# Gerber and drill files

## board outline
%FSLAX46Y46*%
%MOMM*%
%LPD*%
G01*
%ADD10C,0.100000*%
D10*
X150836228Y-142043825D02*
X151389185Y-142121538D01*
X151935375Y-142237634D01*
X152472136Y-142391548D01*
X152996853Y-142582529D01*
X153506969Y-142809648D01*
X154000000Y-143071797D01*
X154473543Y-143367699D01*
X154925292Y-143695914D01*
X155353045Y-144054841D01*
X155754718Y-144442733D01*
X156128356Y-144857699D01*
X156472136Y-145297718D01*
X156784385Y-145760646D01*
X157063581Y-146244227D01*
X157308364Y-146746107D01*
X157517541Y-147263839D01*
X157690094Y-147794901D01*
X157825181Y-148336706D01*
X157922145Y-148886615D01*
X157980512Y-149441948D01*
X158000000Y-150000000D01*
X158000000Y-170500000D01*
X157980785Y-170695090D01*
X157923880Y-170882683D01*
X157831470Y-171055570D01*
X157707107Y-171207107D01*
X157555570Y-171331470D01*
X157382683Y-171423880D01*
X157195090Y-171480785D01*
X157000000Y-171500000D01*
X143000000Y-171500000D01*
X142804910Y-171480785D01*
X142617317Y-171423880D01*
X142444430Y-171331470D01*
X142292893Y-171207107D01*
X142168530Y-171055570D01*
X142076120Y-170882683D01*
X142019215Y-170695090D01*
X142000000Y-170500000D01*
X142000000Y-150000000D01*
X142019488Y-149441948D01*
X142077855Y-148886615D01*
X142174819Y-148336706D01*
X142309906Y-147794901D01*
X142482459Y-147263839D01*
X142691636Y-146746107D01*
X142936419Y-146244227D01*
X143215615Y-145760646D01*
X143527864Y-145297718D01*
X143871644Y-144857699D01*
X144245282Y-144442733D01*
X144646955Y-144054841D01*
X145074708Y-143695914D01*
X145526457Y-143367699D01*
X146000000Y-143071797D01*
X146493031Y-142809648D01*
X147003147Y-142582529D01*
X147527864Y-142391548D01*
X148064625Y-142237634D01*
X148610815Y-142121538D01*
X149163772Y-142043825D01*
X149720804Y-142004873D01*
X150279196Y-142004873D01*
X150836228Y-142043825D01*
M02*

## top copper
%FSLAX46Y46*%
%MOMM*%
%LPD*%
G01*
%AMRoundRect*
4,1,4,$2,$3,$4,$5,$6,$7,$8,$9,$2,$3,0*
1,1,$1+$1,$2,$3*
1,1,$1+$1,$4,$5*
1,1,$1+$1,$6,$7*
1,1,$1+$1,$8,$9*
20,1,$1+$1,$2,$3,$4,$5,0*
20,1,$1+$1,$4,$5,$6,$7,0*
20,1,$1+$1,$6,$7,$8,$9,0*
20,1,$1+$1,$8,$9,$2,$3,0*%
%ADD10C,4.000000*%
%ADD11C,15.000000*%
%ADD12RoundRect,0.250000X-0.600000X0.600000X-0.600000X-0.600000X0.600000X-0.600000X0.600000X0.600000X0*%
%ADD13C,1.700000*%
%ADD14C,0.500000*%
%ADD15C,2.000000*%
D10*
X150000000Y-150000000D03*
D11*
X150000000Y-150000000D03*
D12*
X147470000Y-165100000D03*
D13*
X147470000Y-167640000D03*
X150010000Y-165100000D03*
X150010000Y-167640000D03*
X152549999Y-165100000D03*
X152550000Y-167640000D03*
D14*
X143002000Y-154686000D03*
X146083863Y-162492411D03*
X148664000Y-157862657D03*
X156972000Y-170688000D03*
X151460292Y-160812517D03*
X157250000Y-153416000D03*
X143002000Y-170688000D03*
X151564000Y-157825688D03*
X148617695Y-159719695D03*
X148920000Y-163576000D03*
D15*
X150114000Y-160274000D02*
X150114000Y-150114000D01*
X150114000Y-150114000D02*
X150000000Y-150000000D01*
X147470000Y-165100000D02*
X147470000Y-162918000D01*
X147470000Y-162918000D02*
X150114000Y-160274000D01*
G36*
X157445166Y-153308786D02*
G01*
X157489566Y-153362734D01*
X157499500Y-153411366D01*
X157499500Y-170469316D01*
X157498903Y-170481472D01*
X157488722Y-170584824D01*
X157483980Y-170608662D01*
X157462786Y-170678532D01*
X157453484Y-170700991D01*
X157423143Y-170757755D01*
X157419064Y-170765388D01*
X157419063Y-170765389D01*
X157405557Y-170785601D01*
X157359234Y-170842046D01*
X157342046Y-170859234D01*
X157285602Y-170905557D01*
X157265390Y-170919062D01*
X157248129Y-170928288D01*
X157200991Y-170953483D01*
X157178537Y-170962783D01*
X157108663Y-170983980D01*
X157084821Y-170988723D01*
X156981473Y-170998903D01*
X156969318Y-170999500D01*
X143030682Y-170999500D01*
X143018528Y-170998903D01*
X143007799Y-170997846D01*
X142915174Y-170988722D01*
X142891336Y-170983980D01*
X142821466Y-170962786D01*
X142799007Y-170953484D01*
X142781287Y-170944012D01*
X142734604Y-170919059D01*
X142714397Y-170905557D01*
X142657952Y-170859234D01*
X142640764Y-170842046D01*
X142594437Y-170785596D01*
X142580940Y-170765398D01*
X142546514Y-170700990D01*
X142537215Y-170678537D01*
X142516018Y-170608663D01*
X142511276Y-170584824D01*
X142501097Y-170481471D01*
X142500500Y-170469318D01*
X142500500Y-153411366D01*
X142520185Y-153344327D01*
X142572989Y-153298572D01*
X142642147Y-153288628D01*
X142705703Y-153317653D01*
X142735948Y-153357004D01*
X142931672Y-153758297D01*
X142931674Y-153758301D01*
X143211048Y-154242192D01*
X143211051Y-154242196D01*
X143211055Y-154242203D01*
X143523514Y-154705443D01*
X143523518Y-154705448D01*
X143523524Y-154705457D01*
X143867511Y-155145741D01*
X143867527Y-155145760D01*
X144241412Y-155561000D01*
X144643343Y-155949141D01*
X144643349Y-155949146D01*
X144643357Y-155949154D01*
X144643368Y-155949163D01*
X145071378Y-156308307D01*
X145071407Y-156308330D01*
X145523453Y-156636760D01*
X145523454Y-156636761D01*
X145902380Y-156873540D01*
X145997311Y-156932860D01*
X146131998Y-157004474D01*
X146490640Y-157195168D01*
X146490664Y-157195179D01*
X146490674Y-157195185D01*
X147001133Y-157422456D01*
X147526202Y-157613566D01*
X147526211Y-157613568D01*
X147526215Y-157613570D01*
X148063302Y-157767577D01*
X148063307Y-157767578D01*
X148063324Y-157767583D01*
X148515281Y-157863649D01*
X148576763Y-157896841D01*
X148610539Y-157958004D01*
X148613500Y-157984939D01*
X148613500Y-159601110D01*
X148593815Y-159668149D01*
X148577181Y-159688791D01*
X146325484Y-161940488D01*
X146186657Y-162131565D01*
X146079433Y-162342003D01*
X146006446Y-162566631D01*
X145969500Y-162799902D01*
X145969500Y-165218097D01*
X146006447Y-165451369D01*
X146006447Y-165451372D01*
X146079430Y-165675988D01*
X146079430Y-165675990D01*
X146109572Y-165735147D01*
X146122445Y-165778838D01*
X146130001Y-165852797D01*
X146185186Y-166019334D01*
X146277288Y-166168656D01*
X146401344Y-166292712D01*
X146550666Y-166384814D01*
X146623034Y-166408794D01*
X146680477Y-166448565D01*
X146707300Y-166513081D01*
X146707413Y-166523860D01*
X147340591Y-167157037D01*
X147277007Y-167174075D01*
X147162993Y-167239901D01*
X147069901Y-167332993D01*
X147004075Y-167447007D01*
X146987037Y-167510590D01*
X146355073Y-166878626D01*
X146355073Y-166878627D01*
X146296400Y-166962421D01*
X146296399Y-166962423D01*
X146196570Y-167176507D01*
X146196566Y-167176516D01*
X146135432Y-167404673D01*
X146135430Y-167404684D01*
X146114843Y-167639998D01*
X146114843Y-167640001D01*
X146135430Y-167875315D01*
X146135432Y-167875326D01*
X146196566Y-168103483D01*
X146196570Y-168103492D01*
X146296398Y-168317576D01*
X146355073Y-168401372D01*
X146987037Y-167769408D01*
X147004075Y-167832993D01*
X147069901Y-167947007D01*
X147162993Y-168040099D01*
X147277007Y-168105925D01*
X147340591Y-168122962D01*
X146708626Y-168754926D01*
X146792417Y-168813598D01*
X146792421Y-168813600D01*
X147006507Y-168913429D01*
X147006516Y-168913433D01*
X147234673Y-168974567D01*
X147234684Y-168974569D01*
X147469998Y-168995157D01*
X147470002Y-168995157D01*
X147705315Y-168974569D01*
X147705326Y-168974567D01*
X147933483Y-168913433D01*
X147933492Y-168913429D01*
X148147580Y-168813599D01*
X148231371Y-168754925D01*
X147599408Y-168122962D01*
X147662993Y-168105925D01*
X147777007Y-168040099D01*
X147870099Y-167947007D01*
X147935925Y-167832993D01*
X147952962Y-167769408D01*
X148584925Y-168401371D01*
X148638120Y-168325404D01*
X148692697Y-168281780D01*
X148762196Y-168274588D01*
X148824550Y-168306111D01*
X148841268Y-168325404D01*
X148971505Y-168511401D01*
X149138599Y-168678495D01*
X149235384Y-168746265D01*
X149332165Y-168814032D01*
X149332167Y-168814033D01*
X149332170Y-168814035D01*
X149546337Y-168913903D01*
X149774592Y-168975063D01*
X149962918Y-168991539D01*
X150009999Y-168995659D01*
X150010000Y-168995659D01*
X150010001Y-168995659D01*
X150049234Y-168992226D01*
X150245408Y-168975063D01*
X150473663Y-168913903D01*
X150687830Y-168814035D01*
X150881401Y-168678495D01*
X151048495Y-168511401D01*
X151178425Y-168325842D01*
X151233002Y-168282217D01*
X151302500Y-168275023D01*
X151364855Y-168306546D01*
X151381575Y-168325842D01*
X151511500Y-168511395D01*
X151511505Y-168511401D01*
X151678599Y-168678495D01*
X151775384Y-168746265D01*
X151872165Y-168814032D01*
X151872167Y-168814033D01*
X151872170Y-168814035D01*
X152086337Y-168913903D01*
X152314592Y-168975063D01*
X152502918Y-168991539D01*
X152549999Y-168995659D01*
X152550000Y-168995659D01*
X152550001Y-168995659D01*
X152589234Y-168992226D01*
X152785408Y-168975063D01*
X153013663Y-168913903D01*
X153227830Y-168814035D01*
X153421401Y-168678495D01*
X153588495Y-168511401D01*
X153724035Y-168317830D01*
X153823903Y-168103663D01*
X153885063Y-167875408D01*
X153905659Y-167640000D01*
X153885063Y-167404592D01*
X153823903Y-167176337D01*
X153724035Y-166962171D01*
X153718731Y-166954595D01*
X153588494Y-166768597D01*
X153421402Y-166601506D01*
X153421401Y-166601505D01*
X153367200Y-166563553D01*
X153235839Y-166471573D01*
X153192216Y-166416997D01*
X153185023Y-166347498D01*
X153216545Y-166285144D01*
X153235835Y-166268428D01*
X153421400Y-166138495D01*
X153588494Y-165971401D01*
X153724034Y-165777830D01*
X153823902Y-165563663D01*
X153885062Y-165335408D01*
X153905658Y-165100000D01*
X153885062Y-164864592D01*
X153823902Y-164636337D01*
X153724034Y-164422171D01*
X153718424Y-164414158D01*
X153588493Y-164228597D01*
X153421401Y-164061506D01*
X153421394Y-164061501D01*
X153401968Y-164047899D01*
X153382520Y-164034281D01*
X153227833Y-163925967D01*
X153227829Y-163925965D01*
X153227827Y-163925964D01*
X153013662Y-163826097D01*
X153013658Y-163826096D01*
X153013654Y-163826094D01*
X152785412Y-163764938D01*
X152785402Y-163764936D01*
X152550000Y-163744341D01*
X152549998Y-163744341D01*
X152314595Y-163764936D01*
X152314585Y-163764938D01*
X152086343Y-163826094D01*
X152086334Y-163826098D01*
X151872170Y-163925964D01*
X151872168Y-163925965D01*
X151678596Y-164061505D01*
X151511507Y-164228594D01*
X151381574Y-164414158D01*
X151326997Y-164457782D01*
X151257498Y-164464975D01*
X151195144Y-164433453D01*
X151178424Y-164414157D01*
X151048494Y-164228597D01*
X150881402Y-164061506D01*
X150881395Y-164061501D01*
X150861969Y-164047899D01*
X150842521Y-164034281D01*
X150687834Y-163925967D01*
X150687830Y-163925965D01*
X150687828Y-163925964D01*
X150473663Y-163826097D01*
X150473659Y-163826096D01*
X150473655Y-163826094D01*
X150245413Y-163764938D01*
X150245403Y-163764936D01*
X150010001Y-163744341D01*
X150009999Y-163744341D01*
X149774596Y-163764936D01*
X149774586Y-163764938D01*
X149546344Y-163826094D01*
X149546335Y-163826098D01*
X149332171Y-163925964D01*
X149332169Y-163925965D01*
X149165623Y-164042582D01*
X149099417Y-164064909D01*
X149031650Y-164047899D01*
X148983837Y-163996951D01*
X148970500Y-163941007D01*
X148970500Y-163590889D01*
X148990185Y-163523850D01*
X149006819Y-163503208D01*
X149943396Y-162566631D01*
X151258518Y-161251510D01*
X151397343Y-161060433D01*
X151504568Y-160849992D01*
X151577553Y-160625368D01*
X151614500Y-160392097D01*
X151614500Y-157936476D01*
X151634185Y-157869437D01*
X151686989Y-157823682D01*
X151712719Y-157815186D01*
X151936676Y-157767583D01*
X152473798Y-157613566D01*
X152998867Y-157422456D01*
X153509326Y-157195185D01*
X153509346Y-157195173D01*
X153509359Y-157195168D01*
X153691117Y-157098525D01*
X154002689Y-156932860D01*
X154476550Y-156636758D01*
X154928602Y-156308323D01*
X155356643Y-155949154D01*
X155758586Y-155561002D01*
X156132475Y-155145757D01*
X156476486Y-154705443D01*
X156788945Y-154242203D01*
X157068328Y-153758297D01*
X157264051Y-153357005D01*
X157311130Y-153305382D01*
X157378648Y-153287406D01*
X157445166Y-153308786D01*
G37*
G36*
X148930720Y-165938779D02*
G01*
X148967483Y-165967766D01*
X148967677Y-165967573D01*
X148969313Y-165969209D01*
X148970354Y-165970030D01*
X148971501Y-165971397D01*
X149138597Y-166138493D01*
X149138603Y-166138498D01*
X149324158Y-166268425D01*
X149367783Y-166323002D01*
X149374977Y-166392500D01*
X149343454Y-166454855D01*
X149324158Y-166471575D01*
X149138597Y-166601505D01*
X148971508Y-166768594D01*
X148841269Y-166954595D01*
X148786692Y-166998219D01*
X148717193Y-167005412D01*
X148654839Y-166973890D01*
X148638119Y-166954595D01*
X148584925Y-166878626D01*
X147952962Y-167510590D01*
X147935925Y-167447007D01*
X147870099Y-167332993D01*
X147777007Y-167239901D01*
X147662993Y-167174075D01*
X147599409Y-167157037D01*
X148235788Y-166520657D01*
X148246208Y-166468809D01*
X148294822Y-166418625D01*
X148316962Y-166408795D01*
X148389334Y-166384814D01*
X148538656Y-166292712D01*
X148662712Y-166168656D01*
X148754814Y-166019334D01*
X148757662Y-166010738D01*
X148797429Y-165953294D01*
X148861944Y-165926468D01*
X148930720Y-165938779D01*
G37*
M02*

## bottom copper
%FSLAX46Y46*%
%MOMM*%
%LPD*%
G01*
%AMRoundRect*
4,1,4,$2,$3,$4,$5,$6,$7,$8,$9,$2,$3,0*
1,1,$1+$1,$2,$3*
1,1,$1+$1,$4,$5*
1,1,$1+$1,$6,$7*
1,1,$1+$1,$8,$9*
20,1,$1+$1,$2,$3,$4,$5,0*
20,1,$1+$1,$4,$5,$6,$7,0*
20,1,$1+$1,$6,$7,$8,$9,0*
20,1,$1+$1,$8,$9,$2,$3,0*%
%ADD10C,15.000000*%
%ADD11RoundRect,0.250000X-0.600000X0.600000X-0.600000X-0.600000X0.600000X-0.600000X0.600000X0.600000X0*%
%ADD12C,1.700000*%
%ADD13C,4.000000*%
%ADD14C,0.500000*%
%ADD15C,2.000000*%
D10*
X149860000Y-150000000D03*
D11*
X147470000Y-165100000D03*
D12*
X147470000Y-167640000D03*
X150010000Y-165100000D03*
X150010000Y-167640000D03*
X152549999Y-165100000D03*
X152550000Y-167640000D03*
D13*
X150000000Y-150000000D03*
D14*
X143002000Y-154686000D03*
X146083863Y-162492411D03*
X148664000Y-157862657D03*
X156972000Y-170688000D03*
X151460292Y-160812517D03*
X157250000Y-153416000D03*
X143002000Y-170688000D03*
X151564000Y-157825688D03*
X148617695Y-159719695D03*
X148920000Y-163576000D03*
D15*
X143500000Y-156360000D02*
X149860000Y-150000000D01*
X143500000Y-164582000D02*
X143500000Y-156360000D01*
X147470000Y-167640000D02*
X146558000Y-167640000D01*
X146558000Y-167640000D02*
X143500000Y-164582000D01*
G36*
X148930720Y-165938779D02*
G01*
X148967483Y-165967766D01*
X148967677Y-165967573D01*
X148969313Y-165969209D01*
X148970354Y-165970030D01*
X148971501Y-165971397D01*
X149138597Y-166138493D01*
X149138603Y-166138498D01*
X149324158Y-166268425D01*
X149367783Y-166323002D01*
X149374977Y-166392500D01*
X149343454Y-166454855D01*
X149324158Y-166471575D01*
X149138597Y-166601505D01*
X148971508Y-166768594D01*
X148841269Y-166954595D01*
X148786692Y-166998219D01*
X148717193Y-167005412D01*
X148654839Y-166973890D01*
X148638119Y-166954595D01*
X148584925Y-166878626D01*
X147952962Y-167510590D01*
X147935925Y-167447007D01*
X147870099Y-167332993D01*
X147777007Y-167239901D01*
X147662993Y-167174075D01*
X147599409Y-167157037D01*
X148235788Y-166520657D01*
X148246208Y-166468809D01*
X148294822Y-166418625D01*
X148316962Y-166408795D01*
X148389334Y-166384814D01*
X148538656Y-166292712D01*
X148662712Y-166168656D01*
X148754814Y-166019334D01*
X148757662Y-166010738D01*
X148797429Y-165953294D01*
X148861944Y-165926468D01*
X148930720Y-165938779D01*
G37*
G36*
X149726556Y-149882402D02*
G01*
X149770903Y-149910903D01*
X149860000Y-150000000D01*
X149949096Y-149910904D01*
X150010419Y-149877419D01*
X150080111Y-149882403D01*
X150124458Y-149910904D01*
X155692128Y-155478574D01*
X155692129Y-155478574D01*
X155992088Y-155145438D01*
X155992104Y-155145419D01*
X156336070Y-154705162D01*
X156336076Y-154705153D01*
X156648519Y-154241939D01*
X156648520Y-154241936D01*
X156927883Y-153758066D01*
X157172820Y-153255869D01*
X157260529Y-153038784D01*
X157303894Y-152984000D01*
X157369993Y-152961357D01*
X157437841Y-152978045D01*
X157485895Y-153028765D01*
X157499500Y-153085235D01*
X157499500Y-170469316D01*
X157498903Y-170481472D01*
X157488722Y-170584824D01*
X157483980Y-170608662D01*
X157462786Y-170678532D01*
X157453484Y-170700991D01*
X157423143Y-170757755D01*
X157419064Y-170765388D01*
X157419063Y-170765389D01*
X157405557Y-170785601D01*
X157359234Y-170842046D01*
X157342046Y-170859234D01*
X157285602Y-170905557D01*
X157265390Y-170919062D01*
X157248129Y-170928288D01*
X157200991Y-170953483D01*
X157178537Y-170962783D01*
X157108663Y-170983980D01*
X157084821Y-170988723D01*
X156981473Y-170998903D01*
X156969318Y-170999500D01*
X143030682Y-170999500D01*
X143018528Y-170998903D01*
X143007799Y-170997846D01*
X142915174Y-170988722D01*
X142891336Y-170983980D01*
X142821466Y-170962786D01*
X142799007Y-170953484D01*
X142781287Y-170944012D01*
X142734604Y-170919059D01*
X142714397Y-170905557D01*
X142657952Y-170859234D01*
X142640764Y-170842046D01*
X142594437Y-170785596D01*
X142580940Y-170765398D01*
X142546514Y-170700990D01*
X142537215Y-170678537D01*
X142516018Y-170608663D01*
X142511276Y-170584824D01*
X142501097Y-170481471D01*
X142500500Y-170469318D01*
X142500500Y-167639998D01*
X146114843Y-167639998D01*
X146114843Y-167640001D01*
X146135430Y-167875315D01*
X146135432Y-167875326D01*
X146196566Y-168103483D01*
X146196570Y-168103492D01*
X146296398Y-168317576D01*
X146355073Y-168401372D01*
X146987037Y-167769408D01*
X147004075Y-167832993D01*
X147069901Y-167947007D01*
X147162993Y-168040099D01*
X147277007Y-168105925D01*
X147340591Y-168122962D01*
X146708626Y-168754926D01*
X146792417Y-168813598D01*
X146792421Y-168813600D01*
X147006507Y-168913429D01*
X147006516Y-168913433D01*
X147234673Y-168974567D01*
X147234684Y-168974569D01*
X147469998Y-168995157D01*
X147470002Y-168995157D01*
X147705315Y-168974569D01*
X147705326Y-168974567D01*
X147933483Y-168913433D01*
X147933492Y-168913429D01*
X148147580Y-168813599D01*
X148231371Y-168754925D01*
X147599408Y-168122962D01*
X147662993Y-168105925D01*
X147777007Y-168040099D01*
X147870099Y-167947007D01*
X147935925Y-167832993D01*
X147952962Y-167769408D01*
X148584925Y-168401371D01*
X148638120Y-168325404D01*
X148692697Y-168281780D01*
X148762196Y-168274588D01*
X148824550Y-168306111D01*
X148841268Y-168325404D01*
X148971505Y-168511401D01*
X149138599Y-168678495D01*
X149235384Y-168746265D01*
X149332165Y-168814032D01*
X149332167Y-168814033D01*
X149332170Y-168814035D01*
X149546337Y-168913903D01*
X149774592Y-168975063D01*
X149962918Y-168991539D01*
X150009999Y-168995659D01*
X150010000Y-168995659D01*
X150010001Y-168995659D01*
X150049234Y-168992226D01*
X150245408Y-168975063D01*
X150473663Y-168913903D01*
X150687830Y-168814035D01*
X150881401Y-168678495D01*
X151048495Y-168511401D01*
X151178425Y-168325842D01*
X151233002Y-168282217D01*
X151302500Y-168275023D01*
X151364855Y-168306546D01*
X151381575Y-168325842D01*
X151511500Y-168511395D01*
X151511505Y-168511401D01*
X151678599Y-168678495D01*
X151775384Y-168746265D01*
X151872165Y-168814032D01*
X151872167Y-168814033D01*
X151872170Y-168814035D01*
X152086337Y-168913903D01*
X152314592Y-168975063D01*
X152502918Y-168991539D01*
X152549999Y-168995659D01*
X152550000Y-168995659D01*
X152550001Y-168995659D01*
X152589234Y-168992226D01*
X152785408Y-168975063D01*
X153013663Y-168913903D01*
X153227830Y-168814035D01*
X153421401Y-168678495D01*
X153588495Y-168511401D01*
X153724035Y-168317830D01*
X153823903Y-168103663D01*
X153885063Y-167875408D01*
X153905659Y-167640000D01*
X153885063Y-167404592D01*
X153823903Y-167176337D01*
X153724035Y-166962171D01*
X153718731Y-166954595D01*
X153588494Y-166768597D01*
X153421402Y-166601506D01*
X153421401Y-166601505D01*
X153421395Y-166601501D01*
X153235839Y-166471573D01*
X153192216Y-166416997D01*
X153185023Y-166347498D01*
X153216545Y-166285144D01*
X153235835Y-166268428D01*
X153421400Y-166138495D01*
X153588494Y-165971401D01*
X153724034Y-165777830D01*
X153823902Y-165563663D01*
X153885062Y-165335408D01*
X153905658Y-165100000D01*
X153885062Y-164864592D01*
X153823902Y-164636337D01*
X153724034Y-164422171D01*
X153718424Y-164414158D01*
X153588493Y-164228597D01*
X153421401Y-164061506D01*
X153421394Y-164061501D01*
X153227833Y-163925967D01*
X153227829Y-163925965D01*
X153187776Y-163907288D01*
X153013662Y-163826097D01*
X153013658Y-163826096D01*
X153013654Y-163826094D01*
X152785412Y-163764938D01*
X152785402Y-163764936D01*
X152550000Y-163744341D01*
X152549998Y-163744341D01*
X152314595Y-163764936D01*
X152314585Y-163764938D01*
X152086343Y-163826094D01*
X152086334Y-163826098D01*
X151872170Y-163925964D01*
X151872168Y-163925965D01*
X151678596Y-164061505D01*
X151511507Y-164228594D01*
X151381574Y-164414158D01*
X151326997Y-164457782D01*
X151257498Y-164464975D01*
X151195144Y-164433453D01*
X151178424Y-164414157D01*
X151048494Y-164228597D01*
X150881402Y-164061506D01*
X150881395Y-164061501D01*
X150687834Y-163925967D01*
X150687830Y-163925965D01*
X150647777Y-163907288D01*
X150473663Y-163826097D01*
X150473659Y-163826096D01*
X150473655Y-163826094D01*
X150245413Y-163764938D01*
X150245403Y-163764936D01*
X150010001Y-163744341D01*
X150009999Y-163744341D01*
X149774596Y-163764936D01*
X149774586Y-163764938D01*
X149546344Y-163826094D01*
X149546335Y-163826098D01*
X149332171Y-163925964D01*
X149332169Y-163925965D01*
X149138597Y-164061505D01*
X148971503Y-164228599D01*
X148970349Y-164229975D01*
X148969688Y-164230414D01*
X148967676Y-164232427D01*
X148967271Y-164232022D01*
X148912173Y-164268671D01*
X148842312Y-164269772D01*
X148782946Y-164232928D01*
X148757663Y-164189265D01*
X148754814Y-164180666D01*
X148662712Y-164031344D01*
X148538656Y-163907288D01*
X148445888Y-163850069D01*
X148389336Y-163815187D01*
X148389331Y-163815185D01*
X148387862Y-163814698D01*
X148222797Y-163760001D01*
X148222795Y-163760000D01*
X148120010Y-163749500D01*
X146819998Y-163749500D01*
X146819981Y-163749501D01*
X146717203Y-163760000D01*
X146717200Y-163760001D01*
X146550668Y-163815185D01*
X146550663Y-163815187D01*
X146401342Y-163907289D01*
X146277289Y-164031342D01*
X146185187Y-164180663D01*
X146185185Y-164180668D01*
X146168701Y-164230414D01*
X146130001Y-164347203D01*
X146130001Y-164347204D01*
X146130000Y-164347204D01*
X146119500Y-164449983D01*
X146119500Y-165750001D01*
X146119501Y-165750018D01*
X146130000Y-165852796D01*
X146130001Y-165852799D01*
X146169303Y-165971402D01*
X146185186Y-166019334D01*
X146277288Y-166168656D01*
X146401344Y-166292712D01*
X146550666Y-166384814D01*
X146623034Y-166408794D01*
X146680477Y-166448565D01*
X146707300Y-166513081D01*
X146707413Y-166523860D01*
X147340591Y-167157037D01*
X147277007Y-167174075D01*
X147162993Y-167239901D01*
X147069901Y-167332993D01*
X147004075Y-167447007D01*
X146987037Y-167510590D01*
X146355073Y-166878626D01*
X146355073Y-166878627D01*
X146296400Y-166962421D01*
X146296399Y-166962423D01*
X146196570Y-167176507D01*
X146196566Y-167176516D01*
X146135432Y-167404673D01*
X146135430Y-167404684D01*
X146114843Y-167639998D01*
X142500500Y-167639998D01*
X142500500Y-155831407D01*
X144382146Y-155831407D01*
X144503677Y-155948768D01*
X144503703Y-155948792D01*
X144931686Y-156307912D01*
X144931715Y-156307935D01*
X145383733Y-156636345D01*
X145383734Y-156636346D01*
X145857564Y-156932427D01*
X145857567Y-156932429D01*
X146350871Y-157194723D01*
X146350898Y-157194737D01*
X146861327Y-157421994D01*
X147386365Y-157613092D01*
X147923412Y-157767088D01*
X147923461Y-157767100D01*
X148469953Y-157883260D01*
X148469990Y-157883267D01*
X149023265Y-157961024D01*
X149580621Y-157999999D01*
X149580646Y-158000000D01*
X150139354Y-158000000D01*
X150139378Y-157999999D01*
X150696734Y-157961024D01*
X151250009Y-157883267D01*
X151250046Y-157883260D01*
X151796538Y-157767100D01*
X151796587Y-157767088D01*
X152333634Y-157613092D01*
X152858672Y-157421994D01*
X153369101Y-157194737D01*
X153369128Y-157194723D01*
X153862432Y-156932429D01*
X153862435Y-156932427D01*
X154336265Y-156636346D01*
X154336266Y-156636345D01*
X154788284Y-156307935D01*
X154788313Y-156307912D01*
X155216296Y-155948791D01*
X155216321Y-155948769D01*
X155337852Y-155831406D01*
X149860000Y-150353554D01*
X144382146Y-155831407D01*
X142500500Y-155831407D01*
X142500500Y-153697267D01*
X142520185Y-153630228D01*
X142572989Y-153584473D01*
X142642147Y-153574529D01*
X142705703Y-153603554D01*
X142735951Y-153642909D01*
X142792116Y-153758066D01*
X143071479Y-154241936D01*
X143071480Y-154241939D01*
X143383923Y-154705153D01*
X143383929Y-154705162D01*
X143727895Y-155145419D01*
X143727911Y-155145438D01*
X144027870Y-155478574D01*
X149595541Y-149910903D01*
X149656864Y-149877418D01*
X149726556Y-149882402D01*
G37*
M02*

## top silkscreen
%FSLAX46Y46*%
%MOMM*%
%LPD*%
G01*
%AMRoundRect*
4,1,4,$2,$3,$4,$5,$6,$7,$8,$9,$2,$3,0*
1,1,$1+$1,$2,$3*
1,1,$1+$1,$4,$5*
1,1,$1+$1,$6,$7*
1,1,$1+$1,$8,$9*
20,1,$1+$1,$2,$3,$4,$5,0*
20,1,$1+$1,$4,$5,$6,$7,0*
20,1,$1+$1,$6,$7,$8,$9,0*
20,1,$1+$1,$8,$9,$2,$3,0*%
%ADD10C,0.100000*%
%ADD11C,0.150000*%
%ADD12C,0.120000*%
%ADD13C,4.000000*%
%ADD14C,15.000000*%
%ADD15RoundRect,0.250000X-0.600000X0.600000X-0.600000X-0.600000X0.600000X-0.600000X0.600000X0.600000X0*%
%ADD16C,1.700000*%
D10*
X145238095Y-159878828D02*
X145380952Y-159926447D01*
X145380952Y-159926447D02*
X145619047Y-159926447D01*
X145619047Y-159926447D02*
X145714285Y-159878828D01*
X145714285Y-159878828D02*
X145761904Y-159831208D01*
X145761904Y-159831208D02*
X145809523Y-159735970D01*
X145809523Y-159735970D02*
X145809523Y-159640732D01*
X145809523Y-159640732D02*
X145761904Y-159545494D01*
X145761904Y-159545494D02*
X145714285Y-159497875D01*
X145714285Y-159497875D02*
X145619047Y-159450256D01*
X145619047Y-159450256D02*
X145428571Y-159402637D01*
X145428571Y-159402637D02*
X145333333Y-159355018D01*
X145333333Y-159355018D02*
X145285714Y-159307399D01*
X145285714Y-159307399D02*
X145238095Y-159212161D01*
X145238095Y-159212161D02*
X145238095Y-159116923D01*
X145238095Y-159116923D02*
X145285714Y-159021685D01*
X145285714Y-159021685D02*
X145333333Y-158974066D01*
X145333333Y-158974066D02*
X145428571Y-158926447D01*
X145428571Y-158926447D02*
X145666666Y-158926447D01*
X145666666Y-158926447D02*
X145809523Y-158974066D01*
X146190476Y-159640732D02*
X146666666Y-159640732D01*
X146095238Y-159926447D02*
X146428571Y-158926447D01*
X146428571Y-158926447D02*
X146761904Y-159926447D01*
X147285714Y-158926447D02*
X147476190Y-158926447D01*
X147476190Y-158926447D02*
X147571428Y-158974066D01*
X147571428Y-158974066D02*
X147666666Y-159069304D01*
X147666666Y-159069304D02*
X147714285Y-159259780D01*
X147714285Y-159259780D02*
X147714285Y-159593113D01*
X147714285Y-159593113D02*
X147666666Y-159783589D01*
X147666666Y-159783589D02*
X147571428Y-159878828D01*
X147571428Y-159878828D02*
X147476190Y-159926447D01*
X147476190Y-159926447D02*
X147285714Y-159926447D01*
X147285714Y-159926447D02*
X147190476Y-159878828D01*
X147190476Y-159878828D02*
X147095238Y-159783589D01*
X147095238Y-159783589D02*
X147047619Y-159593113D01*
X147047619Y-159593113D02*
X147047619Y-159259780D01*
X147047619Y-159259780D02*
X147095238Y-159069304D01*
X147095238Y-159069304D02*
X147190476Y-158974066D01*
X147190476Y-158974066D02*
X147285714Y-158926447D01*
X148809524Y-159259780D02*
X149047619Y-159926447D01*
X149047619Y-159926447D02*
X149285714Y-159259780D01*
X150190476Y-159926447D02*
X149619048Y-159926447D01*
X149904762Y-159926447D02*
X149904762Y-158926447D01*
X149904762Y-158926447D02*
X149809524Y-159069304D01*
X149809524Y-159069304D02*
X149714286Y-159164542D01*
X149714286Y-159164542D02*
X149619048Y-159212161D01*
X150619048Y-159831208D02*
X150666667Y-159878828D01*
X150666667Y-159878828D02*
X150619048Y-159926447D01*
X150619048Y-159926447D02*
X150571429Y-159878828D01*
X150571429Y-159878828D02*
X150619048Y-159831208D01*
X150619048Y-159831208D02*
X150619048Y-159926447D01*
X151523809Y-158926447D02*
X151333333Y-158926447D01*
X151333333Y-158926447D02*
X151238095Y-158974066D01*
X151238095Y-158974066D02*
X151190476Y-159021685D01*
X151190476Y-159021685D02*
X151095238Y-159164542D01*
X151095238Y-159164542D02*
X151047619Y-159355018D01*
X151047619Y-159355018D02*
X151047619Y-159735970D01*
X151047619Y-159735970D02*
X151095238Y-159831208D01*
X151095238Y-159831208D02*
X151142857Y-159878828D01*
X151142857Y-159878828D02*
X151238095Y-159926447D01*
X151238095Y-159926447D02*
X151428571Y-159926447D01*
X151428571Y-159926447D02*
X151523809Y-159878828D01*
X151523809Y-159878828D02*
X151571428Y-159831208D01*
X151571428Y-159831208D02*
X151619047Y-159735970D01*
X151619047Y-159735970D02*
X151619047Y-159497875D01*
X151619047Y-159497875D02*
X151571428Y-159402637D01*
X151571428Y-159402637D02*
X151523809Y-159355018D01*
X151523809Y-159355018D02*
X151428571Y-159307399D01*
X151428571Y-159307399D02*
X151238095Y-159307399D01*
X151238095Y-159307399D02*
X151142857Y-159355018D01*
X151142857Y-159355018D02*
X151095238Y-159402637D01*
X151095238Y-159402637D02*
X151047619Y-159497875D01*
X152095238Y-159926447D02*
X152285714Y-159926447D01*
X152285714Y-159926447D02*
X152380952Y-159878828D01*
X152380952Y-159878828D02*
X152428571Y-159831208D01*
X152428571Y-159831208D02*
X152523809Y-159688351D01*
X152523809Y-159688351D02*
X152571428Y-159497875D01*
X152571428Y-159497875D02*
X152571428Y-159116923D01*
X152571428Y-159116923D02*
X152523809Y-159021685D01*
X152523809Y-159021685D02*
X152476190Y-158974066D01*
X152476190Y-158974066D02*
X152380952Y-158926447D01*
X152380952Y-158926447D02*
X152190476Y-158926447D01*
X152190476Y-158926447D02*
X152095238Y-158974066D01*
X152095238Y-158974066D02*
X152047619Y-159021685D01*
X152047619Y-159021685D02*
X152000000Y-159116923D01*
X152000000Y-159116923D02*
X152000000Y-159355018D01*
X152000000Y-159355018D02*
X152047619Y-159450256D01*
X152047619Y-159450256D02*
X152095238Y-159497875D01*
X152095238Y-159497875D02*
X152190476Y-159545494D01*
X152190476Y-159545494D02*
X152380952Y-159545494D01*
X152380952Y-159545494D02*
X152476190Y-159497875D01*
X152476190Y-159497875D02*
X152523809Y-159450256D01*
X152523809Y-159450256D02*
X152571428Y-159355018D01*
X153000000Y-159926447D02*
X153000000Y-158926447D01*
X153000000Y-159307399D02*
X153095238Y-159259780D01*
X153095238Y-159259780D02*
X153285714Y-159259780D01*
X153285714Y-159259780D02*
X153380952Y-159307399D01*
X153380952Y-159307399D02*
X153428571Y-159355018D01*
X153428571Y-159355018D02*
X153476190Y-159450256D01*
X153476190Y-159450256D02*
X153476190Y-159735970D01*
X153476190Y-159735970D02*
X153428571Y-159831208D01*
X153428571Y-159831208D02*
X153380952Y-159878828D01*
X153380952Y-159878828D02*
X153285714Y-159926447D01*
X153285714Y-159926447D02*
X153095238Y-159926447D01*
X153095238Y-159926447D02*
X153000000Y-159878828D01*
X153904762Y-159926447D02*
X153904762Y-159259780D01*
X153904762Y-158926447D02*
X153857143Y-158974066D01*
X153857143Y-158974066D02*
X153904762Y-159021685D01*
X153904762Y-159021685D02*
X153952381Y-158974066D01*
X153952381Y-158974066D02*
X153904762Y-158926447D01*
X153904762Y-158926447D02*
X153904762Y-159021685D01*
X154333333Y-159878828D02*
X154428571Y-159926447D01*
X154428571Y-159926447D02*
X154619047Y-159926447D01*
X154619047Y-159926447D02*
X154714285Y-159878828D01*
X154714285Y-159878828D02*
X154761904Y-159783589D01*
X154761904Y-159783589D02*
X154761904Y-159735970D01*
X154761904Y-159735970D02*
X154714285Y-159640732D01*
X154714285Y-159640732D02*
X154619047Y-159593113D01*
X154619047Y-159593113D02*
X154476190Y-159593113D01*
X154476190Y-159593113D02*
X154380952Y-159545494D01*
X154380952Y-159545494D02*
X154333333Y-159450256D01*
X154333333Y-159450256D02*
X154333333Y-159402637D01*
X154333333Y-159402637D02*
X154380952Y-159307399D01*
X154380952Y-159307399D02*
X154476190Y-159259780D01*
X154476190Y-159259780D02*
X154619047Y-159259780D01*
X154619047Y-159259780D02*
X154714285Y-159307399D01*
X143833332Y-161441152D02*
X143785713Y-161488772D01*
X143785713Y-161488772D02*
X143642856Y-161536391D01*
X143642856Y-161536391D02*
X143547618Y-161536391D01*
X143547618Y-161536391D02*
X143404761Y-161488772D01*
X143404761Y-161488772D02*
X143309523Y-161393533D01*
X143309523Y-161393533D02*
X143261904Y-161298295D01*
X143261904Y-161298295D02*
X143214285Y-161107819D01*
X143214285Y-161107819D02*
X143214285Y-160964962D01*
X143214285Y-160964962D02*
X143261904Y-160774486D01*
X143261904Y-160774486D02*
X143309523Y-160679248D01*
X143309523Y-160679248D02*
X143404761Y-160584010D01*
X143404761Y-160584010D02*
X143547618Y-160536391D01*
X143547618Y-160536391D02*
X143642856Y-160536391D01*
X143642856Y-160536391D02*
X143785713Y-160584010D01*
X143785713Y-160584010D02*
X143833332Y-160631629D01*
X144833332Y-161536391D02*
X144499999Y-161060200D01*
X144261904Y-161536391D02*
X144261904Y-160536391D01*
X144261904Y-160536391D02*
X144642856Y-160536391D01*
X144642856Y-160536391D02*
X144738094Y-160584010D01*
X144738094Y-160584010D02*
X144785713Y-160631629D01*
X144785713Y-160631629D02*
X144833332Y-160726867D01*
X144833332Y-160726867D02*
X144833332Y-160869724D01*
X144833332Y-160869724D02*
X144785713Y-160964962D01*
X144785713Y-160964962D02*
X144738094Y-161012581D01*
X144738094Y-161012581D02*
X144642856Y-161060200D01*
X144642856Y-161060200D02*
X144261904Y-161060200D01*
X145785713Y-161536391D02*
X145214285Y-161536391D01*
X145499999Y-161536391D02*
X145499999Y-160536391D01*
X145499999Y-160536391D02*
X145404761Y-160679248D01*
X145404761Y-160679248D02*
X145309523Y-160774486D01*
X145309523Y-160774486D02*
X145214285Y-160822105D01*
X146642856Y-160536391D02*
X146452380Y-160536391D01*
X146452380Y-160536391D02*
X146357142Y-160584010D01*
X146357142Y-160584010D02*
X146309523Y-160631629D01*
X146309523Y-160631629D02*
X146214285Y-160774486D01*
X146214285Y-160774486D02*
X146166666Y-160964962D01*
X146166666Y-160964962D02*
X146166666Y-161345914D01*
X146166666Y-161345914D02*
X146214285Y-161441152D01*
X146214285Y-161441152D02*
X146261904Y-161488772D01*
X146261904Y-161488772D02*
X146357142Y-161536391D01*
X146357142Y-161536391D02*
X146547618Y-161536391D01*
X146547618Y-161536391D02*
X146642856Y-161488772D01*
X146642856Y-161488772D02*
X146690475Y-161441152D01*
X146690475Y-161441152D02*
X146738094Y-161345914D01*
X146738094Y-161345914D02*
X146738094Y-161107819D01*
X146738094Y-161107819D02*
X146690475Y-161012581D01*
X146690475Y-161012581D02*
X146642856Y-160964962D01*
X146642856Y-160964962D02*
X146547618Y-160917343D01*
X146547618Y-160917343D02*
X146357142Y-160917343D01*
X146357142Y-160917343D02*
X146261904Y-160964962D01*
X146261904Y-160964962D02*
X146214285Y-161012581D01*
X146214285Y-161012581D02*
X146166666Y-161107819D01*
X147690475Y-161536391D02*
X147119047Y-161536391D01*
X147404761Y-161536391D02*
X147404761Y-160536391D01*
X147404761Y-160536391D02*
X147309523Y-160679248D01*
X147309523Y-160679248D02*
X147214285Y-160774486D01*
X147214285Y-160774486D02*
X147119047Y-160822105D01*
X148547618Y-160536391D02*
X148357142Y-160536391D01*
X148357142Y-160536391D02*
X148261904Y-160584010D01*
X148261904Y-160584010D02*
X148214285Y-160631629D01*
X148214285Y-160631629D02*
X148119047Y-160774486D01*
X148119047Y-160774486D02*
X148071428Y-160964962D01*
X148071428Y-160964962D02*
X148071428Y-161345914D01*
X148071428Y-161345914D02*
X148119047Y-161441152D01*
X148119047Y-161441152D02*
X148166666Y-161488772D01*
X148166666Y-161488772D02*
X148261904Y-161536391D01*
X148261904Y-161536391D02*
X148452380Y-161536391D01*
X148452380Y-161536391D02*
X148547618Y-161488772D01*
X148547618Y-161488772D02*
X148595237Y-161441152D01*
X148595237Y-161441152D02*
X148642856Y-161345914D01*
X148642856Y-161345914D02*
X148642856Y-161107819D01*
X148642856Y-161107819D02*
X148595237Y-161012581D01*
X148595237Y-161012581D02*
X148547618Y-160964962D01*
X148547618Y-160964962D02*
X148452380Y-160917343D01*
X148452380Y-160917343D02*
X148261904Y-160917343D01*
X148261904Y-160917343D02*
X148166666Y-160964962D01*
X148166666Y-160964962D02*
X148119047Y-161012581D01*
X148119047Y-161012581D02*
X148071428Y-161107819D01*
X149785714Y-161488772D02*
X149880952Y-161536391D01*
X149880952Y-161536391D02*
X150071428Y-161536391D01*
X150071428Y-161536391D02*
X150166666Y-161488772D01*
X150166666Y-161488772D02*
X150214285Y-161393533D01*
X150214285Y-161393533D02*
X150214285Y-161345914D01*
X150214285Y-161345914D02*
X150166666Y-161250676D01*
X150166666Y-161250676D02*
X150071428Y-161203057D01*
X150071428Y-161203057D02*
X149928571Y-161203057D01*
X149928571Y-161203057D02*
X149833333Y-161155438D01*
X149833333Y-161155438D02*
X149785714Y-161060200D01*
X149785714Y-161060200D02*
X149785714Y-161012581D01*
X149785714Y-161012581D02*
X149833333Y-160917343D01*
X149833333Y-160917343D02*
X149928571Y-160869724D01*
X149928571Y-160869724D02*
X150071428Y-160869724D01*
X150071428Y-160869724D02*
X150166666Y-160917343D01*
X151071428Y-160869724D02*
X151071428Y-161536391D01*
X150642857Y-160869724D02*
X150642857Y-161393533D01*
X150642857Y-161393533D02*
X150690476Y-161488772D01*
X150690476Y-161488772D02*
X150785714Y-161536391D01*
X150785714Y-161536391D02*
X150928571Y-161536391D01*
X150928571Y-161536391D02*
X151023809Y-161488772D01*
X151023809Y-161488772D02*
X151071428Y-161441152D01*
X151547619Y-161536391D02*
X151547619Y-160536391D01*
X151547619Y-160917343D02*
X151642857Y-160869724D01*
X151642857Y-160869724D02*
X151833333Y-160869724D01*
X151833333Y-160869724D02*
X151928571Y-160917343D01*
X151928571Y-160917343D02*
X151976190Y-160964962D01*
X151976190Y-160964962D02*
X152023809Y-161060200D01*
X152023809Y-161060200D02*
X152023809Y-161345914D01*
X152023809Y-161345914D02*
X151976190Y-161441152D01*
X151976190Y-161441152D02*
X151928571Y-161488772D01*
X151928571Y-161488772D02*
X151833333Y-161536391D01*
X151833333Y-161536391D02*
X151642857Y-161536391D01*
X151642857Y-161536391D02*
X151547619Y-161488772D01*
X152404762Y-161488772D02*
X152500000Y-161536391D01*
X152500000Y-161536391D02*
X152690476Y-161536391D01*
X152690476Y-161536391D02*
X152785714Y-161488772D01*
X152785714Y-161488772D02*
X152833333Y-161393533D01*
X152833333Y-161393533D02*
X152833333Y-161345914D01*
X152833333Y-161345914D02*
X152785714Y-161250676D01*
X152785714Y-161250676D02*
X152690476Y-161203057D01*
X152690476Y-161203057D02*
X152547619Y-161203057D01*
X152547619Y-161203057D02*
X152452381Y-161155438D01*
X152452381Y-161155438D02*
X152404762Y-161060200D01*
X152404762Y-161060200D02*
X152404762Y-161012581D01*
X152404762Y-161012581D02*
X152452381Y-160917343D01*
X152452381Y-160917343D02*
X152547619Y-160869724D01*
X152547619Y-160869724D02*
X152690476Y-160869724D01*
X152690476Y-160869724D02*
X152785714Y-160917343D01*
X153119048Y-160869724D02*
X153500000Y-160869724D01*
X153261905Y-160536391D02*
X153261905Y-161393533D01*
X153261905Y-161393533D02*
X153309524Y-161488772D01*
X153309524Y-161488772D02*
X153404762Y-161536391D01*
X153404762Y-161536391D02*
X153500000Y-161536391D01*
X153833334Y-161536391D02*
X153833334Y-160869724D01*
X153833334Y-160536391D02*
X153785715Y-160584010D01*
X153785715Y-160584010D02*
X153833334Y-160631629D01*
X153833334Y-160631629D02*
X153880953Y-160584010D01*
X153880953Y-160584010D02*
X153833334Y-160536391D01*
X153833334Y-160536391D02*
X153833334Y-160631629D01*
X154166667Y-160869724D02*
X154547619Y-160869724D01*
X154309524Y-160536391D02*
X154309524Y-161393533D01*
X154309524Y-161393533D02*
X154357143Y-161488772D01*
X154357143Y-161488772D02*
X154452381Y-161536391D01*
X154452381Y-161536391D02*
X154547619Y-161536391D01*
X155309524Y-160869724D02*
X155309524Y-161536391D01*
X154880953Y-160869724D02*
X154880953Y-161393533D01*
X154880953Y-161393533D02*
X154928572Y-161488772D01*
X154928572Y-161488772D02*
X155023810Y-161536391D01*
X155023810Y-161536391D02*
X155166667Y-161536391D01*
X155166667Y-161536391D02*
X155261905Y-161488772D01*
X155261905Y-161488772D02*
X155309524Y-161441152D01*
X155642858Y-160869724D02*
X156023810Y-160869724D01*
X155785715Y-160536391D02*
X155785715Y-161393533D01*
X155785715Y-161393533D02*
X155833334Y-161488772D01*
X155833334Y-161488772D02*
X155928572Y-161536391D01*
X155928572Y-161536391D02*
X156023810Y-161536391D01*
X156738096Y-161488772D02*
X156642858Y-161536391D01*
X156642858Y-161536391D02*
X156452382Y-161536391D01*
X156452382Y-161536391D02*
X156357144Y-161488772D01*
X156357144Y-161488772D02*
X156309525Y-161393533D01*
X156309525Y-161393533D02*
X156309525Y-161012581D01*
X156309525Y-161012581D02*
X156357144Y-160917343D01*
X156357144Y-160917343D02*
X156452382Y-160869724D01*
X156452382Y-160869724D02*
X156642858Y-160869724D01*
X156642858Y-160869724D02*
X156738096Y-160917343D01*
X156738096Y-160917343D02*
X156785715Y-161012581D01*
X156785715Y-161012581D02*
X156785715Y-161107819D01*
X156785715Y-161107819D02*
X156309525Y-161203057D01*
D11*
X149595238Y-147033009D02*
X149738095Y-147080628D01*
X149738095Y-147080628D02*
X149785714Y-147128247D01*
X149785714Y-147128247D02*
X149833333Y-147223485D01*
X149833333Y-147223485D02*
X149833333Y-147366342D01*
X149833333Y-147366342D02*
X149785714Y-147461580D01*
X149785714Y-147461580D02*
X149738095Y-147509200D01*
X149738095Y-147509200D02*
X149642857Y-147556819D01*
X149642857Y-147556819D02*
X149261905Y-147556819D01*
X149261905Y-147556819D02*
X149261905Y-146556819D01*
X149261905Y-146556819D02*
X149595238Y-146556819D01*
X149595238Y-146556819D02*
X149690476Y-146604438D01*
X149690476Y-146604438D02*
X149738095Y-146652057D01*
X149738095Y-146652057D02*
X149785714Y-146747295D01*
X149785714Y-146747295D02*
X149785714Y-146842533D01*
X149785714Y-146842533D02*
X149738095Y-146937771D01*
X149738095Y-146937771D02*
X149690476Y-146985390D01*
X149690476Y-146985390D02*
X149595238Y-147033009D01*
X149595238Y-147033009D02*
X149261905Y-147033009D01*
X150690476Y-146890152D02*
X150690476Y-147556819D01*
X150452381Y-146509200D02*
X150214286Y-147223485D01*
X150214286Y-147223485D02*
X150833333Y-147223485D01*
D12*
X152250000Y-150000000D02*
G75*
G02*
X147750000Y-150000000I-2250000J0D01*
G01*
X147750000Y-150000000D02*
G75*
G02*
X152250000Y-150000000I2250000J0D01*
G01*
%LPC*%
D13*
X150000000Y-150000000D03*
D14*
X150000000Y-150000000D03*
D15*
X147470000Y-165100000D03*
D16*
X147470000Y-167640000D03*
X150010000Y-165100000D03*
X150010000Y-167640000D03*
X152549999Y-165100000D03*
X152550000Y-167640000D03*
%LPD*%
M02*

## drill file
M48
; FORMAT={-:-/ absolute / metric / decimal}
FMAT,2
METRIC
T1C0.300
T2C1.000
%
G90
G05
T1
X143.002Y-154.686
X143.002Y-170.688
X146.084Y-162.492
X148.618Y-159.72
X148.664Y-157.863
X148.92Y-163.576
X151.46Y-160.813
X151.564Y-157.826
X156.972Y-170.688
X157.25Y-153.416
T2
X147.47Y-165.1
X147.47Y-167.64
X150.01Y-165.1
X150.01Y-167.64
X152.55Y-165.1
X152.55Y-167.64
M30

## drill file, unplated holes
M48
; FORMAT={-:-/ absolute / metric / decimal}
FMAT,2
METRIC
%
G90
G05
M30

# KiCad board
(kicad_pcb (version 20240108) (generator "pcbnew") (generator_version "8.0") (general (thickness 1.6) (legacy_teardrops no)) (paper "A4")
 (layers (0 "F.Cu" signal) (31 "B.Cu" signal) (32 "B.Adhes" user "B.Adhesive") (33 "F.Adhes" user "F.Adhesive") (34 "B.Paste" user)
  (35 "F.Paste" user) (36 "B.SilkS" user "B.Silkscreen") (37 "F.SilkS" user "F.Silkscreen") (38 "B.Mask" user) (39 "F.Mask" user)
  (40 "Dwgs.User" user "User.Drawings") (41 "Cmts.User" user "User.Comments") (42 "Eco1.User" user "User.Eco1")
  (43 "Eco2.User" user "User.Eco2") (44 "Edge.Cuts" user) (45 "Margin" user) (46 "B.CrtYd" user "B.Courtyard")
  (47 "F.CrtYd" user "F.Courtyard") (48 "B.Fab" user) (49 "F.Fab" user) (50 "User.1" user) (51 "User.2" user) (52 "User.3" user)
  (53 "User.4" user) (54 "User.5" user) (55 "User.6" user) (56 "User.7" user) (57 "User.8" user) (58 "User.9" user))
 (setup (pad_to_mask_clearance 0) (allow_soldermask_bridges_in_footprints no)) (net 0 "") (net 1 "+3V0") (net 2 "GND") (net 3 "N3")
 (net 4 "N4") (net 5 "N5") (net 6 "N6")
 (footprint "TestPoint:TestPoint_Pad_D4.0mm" (layer "F.Cu") (at 150 150)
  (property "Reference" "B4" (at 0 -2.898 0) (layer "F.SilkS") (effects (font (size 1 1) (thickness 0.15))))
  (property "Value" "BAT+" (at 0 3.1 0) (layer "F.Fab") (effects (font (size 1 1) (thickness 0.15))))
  (fp_circle (center 0 0) (end 0 2.25) (stroke (width 0.12) (type solid)) (fill none) (layer "F.SilkS"))
  (pad "1" smd circle (at 0 0) (size 4 4) (layers "F.Cu" "F.Mask") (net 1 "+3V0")))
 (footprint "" (layer "B.Cu") (at 150 150 180)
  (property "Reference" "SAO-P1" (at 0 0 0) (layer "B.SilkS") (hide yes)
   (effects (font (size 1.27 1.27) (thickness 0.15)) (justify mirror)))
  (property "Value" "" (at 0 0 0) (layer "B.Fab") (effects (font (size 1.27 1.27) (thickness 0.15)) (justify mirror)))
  (pad "1" smd circle (at 0 0) (size 15 15) (layers "F.Cu" "F.Mask") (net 1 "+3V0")))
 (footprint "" (layer "B.Cu") (at 150 150 180)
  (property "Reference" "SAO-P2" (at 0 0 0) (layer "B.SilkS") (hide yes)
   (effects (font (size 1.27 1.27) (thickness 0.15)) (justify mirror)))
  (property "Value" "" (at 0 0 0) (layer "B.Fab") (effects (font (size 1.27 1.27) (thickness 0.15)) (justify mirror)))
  (pad "1" smd circle (at 0.14 0 180) (size 15 15) (layers "B.Cu" "B.Mask") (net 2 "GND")))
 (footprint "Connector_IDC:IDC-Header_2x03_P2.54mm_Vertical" (layer "B.Cu") (at 147.47 165.1 -90)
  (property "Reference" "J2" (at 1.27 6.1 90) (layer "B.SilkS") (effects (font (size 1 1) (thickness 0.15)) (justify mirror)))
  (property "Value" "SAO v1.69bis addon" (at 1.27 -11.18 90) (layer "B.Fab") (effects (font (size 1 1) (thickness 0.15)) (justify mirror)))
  (pad "1" thru_hole roundrect (at 0 0 270) (size 1.7 1.7) (drill 1) (layers "*.Cu" "*.Mask") (remove_unused_layers no)
   (roundrect_rratio 0.147059) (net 1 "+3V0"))
  (pad "2" thru_hole circle (at 2.54 0 270) (size 1.7 1.7) (drill 1) (layers "*.Cu" "*.Mask") (remove_unused_layers no) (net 2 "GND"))
  (pad "3" thru_hole circle (at 0 -2.54 270) (size 1.7 1.7) (drill 1) (layers "*.Cu" "*.Mask") (remove_unused_layers no) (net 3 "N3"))
  (pad "4" thru_hole circle (at 2.54 -2.54 270) (size 1.7 1.7) (drill 1) (layers "*.Cu" "*.Mask") (remove_unused_layers no) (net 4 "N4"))
  (pad "5" thru_hole circle (at 0 -5.079999 270) (size 1.7 1.7) (drill 1) (layers "*.Cu" "*.Mask") (remove_unused_layers no) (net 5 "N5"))
  (pad "6" thru_hole circle (at 2.54 -5.08 270) (size 1.7 1.7) (drill 1) (layers "*.Cu" "*.Mask") (remove_unused_layers no) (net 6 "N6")))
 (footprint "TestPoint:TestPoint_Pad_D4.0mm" (layer "B.Cu") (at 150 150 180)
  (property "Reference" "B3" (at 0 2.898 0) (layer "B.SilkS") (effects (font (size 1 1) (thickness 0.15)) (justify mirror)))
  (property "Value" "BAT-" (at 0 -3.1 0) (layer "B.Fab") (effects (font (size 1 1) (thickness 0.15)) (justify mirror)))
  (pad "1" smd circle (at 0 0 180) (size 4 4) (layers "B.Cu" "B.Mask") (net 2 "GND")))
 (gr_poly
  (pts (xy 149.163772 142.043825) (xy 149.720804 142.004873) (xy 150.279196 142.004873) (xy 150.836228 142.043825)
   (xy 151.389185 142.121538) (xy 151.935375 142.237634) (xy 152.472136 142.391548) (xy 152.996853 142.582529) (xy 153.506969 142.809648)
   (xy 154 143.071797) (xy 154.473543 143.367699) (xy 154.925292 143.695914) (xy 155.353045 144.054841) (xy 155.754718 144.442733)
   (xy 156.128356 144.857699) (xy 156.472136 145.297718) (xy 156.784385 145.760646) (xy 157.063581 146.244227) (xy 157.308364 146.746107)
   (xy 157.517541 147.263839) (xy 157.690094 147.794901) (xy 157.825181 148.336706) (xy 157.922145 148.886615) (xy 157.980512 149.441948)
   (xy 158 150) (xy 158 170.5) (xy 157.980785 170.69509) (xy 157.92388 170.882683) (xy 157.83147 171.05557) (xy 157.707107 171.207107)
   (xy 157.55557 171.33147) (xy 157.382683 171.42388) (xy 157.19509 171.480785) (xy 157 171.5) (xy 143 171.5) (xy 142.80491 171.480785)
   (xy 142.617317 171.42388) (xy 142.44443 171.33147) (xy 142.292893 171.207107) (xy 142.16853 171.05557) (xy 142.07612 170.882683)
   (xy 142.019215 170.69509) (xy 142 170.5) (xy 142 150) (xy 142.019488 149.441948) (xy 142.077855 148.886615) (xy 142.174819 148.336706)
   (xy 142.309906 147.794901) (xy 142.482459 147.263839) (xy 142.691636 146.746107) (xy 142.936419 146.244227) (xy 143.215615 145.760646)
   (xy 143.527864 145.297718) (xy 143.871644 144.857699) (xy 144.245282 144.442733) (xy 144.646955 144.054841) (xy 145.074708 143.695914)
   (xy 145.526457 143.367699) (xy 146 143.071797) (xy 146.493031 142.809648) (xy 147.003147 142.582529) (xy 147.527864 142.391548)
   (xy 148.064625 142.237634) (xy 148.610815 142.121538))
  (stroke (width 0.1) (type solid)) (fill none) (layer "Edge.Cuts"))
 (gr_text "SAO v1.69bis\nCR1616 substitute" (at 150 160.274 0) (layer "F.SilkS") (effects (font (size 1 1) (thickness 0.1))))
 (via (at 146.083863 162.492411) (size 0.5) (drill 0.3) (layers "F.Cu" "B.Cu") (free yes) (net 2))
 (via (at 148.664 157.862657) (size 0.5) (drill 0.3) (layers "F.Cu" "B.Cu") (free yes) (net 2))
 (via (at 156.972 170.688) (size 0.5) (drill 0.3) (layers "F.Cu" "B.Cu") (free yes) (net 2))
 (via (at 151.460292 160.812517) (size 0.5) (drill 0.3) (layers "F.Cu" "B.Cu") (free yes) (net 2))
 (via (at 157.25 153.416) (size 0.5) (drill 0.3) (layers "F.Cu" "B.Cu") (free yes) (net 2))
 (via (at 143.002 170.688) (size 0.5) (drill 0.3) (layers "F.Cu" "B.Cu") (free yes) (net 2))
 (via (at 151.564 157.825688) (size 0.5) (drill 0.3) (layers "F.Cu" "B.Cu") (free yes) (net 2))
 (via (at 143.002 154.686) (size 0.5) (drill 0.3) (layers "F.Cu" "B.Cu") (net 2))
 (via (at 148.617695 159.719695) (size 0.5) (drill 0.3) (layers "F.Cu" "B.Cu") (free yes) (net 2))
 (via (at 148.92 163.576) (size 0.5) (drill 0.3) (layers "F.Cu" "B.Cu") (free yes) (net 2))
 (segment (start 143.5 156.36) (end 149.86 150) (width 2) (layer "B.Cu") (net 2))
 (segment (start 143.5 164.582) (end 143.5 156.36) (width 2) (layer "B.Cu") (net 2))
 (segment (start 147.47 167.64) (end 146.558 167.64) (width 2) (layer "B.Cu") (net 2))
 (segment (start 146.558 167.64) (end 143.5 164.582) (width 2) (layer "B.Cu") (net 2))
 (segment (start 150.114 160.274) (end 150.114 150.114) (width 2) (layer "F.Cu") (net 1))
 (segment (start 150.114 150.114) (end 150 150) (width 2) (layer "F.Cu") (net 1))
 (segment (start 147.47 165.1) (end 147.47 162.918) (width 2) (layer "F.Cu") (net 1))
 (segment (start 147.47 162.918) (end 150.114 160.274) (width 2) (layer "F.Cu") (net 1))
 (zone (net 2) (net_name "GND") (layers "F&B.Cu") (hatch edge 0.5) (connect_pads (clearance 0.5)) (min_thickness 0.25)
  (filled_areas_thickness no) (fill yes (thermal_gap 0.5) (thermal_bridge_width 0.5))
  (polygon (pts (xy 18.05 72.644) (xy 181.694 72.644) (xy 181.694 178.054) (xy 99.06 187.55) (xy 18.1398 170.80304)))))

